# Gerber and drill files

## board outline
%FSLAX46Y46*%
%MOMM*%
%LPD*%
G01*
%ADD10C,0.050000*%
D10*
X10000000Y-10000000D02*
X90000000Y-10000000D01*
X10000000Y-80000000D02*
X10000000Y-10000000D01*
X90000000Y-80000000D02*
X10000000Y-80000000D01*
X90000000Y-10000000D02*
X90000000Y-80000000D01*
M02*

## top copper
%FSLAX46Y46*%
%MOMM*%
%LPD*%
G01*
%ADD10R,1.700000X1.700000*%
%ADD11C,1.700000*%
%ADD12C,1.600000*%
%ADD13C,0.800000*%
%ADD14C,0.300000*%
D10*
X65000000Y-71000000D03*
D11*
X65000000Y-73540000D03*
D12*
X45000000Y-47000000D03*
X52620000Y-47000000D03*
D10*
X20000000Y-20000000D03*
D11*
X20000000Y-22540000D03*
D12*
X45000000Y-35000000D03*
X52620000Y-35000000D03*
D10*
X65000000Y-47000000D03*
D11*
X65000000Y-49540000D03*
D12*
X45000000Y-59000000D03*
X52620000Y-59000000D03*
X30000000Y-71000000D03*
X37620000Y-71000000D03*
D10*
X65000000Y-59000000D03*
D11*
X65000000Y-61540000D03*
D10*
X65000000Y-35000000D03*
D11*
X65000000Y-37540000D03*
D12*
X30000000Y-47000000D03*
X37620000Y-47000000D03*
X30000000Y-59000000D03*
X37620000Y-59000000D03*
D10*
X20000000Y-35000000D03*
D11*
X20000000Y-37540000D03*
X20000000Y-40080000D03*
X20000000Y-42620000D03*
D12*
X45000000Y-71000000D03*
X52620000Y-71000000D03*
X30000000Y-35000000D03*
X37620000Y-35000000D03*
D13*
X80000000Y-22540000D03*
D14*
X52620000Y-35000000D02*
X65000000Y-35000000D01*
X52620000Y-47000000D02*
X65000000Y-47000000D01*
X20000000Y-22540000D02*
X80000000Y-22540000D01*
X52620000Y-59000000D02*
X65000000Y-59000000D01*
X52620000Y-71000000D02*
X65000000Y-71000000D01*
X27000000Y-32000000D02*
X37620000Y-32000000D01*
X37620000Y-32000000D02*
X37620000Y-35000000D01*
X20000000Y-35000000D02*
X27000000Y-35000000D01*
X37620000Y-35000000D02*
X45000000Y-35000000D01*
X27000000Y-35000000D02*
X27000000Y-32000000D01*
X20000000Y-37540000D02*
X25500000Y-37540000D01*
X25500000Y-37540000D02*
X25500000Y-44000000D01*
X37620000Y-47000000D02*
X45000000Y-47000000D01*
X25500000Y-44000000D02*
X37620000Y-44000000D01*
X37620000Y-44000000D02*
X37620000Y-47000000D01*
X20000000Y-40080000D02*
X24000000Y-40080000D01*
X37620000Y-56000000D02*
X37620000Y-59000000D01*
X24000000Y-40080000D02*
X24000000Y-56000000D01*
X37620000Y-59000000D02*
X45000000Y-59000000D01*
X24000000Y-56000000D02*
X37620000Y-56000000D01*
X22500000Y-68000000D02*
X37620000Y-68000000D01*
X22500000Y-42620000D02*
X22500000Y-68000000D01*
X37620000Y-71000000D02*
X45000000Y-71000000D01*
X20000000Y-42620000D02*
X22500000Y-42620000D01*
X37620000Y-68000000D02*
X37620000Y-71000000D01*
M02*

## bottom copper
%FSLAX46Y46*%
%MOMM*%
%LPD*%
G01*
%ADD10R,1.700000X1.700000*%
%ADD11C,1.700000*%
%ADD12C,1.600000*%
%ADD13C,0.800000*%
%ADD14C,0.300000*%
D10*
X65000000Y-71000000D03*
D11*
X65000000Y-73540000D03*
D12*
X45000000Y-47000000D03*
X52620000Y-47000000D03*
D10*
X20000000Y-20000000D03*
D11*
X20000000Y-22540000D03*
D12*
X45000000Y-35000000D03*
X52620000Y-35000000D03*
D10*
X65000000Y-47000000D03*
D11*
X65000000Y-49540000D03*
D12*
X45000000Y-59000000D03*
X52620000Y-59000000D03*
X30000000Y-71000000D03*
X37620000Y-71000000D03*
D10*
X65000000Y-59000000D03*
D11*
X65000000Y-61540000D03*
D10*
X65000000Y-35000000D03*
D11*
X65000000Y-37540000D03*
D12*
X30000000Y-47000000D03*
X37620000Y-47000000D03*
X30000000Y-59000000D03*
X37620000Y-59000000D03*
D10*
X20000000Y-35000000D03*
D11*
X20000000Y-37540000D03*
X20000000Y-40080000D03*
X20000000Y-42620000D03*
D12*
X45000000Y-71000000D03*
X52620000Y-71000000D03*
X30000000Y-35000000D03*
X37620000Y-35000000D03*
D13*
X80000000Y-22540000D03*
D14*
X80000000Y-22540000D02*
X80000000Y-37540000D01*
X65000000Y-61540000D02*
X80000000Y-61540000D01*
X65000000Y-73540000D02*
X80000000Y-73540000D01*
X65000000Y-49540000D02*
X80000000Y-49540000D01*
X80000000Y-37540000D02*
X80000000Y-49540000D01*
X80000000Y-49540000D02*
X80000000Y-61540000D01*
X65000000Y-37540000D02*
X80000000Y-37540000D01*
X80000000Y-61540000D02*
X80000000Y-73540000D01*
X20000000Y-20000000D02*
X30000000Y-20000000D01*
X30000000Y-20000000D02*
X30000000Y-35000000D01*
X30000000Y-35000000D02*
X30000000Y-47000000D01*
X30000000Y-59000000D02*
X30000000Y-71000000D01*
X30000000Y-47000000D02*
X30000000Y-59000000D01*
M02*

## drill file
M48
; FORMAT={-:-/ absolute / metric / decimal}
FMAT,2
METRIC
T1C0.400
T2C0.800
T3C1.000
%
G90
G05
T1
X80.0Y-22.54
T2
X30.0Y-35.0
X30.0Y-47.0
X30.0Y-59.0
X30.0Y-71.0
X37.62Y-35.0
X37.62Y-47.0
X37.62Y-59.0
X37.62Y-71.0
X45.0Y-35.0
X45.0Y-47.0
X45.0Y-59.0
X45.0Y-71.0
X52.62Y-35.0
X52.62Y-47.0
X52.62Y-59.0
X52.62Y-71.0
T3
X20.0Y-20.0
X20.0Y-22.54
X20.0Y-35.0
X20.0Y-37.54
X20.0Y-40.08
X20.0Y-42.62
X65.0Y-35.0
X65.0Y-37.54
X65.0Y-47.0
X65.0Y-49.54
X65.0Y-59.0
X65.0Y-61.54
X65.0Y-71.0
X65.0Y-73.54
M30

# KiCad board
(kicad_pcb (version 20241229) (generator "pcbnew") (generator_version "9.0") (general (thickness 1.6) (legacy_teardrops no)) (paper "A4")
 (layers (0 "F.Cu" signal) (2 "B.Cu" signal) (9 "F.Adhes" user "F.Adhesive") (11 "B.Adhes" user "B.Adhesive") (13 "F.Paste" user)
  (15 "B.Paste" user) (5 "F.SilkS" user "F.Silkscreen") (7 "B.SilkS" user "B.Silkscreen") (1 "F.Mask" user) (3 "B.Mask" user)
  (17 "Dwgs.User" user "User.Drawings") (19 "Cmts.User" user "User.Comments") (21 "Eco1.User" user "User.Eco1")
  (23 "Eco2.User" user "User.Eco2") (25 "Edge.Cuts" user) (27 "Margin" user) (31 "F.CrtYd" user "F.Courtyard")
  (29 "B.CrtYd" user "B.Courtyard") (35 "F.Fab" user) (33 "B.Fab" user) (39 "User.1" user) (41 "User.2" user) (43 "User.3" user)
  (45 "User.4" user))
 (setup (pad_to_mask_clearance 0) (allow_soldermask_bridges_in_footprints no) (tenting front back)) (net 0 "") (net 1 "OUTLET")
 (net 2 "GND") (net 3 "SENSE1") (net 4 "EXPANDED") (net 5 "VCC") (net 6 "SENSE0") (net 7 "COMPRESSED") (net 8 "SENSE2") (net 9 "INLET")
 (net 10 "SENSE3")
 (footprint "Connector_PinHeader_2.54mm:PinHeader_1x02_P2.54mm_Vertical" (layer "F.Cu") (at 65 71)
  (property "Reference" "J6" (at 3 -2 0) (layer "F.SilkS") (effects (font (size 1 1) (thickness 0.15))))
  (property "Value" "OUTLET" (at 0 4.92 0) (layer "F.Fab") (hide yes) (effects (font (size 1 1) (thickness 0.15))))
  (pad "1" thru_hole rect (at 0 0) (size 1.7 1.7) (drill 1) (layers "*.Cu" "*.Mask") (remove_unused_layers no) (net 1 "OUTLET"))
  (pad "2" thru_hole circle (at 0 2.54) (size 1.7 1.7) (drill 1) (layers "*.Cu" "*.Mask") (remove_unused_layers no) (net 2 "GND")))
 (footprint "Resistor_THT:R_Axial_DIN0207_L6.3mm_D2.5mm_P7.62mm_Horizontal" (layer "F.Cu") (at 45 47)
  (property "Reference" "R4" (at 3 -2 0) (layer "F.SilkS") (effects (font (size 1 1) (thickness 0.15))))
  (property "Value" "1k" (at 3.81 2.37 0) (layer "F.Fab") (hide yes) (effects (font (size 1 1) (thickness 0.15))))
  (pad "1" thru_hole circle (at 0 0) (size 1.6 1.6) (drill 0.8) (layers "*.Cu" "*.Mask") (remove_unused_layers no) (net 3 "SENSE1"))
  (pad "2" thru_hole circle (at 7.62 0) (size 1.6 1.6) (drill 0.8) (layers "*.Cu" "*.Mask") (remove_unused_layers no) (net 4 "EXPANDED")))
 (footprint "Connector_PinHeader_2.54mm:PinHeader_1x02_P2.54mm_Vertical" (layer "F.Cu") (at 20 20)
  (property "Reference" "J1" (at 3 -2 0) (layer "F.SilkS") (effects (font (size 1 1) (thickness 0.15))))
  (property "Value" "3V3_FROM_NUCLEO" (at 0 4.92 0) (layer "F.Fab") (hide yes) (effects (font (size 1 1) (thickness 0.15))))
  (pad "1" thru_hole rect (at 0 0) (size 1.7 1.7) (drill 1) (layers "*.Cu" "*.Mask") (remove_unused_layers no) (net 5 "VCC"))
  (pad "2" thru_hole circle (at 0 2.54) (size 1.7 1.7) (drill 1) (layers "*.Cu" "*.Mask") (remove_unused_layers no) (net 2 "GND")))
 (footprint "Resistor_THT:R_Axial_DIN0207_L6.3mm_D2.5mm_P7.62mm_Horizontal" (layer "F.Cu") (at 45 35)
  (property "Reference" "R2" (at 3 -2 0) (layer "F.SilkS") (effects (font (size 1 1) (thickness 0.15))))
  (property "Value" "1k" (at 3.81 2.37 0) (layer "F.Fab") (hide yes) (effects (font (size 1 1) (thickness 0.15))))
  (pad "1" thru_hole circle (at 0 0) (size 1.6 1.6) (drill 0.8) (layers "*.Cu" "*.Mask") (remove_unused_layers no) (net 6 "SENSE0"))
  (pad "2" thru_hole circle (at 7.62 0) (size 1.6 1.6) (drill 0.8) (layers "*.Cu" "*.Mask") (remove_unused_layers no) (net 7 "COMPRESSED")))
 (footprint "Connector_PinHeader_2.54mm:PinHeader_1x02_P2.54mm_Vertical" (layer "F.Cu") (at 65 47)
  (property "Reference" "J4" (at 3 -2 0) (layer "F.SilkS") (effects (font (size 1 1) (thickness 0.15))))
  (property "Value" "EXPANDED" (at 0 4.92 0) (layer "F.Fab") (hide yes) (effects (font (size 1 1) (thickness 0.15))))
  (pad "1" thru_hole rect (at 0 0) (size 1.7 1.7) (drill 1) (layers "*.Cu" "*.Mask") (remove_unused_layers no) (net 4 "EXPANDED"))
  (pad "2" thru_hole circle (at 0 2.54) (size 1.7 1.7) (drill 1) (layers "*.Cu" "*.Mask") (remove_unused_layers no) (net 2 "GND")))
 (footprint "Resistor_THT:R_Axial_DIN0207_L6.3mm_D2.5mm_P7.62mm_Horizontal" (layer "F.Cu") (at 45 59)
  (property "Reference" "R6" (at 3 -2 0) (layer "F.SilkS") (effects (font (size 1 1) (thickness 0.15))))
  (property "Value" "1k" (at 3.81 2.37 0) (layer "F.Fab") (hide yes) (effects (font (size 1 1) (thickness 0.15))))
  (pad "1" thru_hole circle (at 0 0) (size 1.6 1.6) (drill 0.8) (layers "*.Cu" "*.Mask") (remove_unused_layers no) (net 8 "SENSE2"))
  (pad "2" thru_hole circle (at 7.62 0) (size 1.6 1.6) (drill 0.8) (layers "*.Cu" "*.Mask") (remove_unused_layers no) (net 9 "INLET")))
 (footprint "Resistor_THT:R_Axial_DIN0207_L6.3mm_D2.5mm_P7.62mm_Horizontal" (layer "F.Cu") (at 30 71)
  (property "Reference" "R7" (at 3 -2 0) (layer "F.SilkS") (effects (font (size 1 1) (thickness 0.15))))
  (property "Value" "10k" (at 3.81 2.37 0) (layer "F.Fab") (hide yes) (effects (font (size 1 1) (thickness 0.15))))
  (pad "1" thru_hole circle (at 0 0) (size 1.6 1.6) (drill 0.8) (layers "*.Cu" "*.Mask") (remove_unused_layers no) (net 5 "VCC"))
  (pad "2" thru_hole circle (at 7.62 0) (size 1.6 1.6) (drill 0.8) (layers "*.Cu" "*.Mask") (remove_unused_layers no) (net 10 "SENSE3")))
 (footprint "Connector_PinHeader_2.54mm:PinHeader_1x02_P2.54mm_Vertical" (layer "F.Cu") (at 65 59)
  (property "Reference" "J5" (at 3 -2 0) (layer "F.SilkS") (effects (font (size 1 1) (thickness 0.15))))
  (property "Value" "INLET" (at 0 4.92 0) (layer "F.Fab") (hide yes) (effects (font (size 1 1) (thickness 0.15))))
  (pad "1" thru_hole rect (at 0 0) (size 1.7 1.7) (drill 1) (layers "*.Cu" "*.Mask") (remove_unused_layers no) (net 9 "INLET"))
  (pad "2" thru_hole circle (at 0 2.54) (size 1.7 1.7) (drill 1) (layers "*.Cu" "*.Mask") (remove_unused_layers no) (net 2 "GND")))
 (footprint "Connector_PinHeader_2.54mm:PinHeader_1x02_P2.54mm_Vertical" (layer "F.Cu") (at 65 35)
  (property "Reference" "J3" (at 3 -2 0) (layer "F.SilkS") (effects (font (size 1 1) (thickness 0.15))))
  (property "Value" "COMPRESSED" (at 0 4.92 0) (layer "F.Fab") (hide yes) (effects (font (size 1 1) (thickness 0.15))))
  (pad "1" thru_hole rect (at 0 0) (size 1.7 1.7) (drill 1) (layers "*.Cu" "*.Mask") (remove_unused_layers no) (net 7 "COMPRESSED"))
  (pad "2" thru_hole circle (at 0 2.54) (size 1.7 1.7) (drill 1) (layers "*.Cu" "*.Mask") (remove_unused_layers no) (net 2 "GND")))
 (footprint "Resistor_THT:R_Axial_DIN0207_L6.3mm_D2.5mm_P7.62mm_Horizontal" (layer "F.Cu") (at 30 47)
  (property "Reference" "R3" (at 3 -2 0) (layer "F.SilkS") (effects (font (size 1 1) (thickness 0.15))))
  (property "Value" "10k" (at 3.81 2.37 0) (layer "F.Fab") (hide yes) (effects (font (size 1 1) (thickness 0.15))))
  (pad "1" thru_hole circle (at 0 0) (size 1.6 1.6) (drill 0.8) (layers "*.Cu" "*.Mask") (remove_unused_layers no) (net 5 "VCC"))
  (pad "2" thru_hole circle (at 7.62 0) (size 1.6 1.6) (drill 0.8) (layers "*.Cu" "*.Mask") (remove_unused_layers no) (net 3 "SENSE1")))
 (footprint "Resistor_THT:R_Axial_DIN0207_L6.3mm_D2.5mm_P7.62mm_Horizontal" (layer "F.Cu") (at 30 59)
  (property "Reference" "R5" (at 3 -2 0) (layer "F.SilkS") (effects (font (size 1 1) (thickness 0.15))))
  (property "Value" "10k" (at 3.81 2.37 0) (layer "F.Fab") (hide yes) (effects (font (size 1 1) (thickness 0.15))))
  (pad "1" thru_hole circle (at 0 0) (size 1.6 1.6) (drill 0.8) (layers "*.Cu" "*.Mask") (remove_unused_layers no) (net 5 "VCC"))
  (pad "2" thru_hole circle (at 7.62 0) (size 1.6 1.6) (drill 0.8) (layers "*.Cu" "*.Mask") (remove_unused_layers no) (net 8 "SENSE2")))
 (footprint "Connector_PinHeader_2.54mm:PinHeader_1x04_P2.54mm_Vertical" (layer "F.Cu") (at 20 35)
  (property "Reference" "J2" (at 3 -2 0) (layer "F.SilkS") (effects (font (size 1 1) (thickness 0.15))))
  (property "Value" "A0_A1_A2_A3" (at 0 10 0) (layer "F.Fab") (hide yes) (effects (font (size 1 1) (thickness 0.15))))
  (pad "1" thru_hole rect (at 0 0) (size 1.7 1.7) (drill 1) (layers "*.Cu" "*.Mask") (remove_unused_layers no) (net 6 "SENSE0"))
  (pad "2" thru_hole circle (at 0 2.54) (size 1.7 1.7) (drill 1) (layers "*.Cu" "*.Mask") (remove_unused_layers no) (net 3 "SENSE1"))
  (pad "3" thru_hole circle (at 0 5.08) (size 1.7 1.7) (drill 1) (layers "*.Cu" "*.Mask") (remove_unused_layers no) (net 8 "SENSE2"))
  (pad "4" thru_hole circle (at 0 7.62) (size 1.7 1.7) (drill 1) (layers "*.Cu" "*.Mask") (remove_unused_layers no) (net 10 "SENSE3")))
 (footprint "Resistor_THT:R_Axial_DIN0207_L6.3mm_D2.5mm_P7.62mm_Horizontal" (layer "F.Cu") (at 45 71)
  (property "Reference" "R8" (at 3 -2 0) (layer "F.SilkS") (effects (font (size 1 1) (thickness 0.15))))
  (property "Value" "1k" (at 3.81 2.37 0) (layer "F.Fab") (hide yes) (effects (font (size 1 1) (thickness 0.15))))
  (pad "1" thru_hole circle (at 0 0) (size 1.6 1.6) (drill 0.8) (layers "*.Cu" "*.Mask") (remove_unused_layers no) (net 10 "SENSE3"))
  (pad "2" thru_hole circle (at 7.62 0) (size 1.6 1.6) (drill 0.8) (layers "*.Cu" "*.Mask") (remove_unused_layers no) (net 1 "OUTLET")))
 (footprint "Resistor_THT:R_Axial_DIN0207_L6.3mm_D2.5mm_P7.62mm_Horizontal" (layer "F.Cu") (at 30 35)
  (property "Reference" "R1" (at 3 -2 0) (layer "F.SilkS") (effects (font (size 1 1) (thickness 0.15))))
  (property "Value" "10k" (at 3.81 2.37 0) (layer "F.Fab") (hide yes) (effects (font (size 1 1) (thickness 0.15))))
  (pad "1" thru_hole circle (at 0 0) (size 1.6 1.6) (drill 0.8) (layers "*.Cu" "*.Mask") (remove_unused_layers no) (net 5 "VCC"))
  (pad "2" thru_hole circle (at 7.62 0) (size 1.6 1.6) (drill 0.8) (layers "*.Cu" "*.Mask") (remove_unused_layers no) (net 6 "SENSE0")))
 (gr_line (start 10 10) (end 90 10) (stroke (width 0.05) (type default)) (layer "Edge.Cuts"))
 (gr_line (start 10 80) (end 10 10) (stroke (width 0.05) (type default)) (layer "Edge.Cuts"))
 (gr_line (start 90 80) (end 10 80) (stroke (width 0.05) (type default)) (layer "Edge.Cuts"))
 (gr_line (start 90 10) (end 90 80) (stroke (width 0.05) (type default)) (layer "Edge.Cuts"))
 (segment (start 52.62 35) (end 65 35) (width 0.3) (layer "F.Cu") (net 7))
 (segment (start 52.62 47) (end 65 47) (width 0.3) (layer "F.Cu") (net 4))
 (segment (start 20 22.54) (end 80 22.54) (width 0.3) (layer "F.Cu") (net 2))
 (via (at 80 22.54) (size 0.8) (drill 0.4) (layers "F.Cu" "B.Cu") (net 2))
 (segment (start 80 22.54) (end 80 37.54) (width 0.3) (layer "B.Cu") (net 2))
 (segment (start 65 61.54) (end 80 61.54) (width 0.3) (layer "B.Cu") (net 2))
 (segment (start 65 73.54) (end 80 73.54) (width 0.3) (layer "B.Cu") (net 2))
 (segment (start 65 49.54) (end 80 49.54) (width 0.3) (layer "B.Cu") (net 2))
 (segment (start 80 37.54) (end 80 49.54) (width 0.3) (layer "B.Cu") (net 2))
 (segment (start 80 49.54) (end 80 61.54) (width 0.3) (layer "B.Cu") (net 2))
 (segment (start 65 37.54) (end 80 37.54) (width 0.3) (layer "B.Cu") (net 2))
 (segment (start 80 61.54) (end 80 73.54) (width 0.3) (layer "B.Cu") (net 2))
 (segment (start 52.62 59) (end 65 59) (width 0.3) (layer "F.Cu") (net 9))
 (segment (start 52.62 71) (end 65 71) (width 0.3) (layer "F.Cu") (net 1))
 (segment (start 27 32) (end 37.62 32) (width 0.3) (layer "F.Cu") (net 6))
 (segment (start 37.62 32) (end 37.62 35) (width 0.3) (layer "F.Cu") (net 6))
 (segment (start 20 35) (end 27 35) (width 0.3) (layer "F.Cu") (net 6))
 (segment (start 37.62 35) (end 45 35) (width 0.3) (layer "F.Cu") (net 6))
 (segment (start 27 35) (end 27 32) (width 0.3) (layer "F.Cu") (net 6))
 (segment (start 20 37.54) (end 25.5 37.54) (width 0.3) (layer "F.Cu") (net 3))
 (segment (start 25.5 37.54) (end 25.5 44) (width 0.3) (layer "F.Cu") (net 3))
 (segment (start 37.62 47) (end 45 47) (width 0.3) (layer "F.Cu") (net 3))
 (segment (start 25.5 44) (end 37.62 44) (width 0.3) (layer "F.Cu") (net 3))
 (segment (start 37.62 44) (end 37.62 47) (width 0.3) (layer "F.Cu") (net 3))
 (segment (start 20 40.08) (end 24 40.08) (width 0.3) (layer "F.Cu") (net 8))
 (segment (start 37.62 56) (end 37.62 59) (width 0.3) (layer "F.Cu") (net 8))
 (segment (start 24 40.08) (end 24 56) (width 0.3) (layer "F.Cu") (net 8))
 (segment (start 37.62 59) (end 45 59) (width 0.3) (layer "F.Cu") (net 8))
 (segment (start 24 56) (end 37.62 56) (width 0.3) (layer "F.Cu") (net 8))
 (segment (start 22.5 68) (end 37.62 68) (width 0.3) (layer "F.Cu") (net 10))
 (segment (start 22.5 42.62) (end 22.5 68) (width 0.3) (layer "F.Cu") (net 10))
 (segment (start 37.62 71) (end 45 71) (width 0.3) (layer "F.Cu") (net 10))
 (segment (start 20 42.62) (end 22.5 42.62) (width 0.3) (layer "F.Cu") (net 10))
 (segment (start 37.62 68) (end 37.62 71) (width 0.3) (layer "F.Cu") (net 10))
 (segment (start 20 20) (end 30 20) (width 0.3) (layer "B.Cu") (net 5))
 (segment (start 30 20) (end 30 35) (width 0.3) (layer "B.Cu") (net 5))
 (segment (start 30 35) (end 30 47) (width 0.3) (layer "B.Cu") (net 5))
 (segment (start 30 59) (end 30 71) (width 0.3) (layer "B.Cu") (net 5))
 (segment (start 30 47) (end 30 59) (width 0.3) (layer "B.Cu") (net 5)))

